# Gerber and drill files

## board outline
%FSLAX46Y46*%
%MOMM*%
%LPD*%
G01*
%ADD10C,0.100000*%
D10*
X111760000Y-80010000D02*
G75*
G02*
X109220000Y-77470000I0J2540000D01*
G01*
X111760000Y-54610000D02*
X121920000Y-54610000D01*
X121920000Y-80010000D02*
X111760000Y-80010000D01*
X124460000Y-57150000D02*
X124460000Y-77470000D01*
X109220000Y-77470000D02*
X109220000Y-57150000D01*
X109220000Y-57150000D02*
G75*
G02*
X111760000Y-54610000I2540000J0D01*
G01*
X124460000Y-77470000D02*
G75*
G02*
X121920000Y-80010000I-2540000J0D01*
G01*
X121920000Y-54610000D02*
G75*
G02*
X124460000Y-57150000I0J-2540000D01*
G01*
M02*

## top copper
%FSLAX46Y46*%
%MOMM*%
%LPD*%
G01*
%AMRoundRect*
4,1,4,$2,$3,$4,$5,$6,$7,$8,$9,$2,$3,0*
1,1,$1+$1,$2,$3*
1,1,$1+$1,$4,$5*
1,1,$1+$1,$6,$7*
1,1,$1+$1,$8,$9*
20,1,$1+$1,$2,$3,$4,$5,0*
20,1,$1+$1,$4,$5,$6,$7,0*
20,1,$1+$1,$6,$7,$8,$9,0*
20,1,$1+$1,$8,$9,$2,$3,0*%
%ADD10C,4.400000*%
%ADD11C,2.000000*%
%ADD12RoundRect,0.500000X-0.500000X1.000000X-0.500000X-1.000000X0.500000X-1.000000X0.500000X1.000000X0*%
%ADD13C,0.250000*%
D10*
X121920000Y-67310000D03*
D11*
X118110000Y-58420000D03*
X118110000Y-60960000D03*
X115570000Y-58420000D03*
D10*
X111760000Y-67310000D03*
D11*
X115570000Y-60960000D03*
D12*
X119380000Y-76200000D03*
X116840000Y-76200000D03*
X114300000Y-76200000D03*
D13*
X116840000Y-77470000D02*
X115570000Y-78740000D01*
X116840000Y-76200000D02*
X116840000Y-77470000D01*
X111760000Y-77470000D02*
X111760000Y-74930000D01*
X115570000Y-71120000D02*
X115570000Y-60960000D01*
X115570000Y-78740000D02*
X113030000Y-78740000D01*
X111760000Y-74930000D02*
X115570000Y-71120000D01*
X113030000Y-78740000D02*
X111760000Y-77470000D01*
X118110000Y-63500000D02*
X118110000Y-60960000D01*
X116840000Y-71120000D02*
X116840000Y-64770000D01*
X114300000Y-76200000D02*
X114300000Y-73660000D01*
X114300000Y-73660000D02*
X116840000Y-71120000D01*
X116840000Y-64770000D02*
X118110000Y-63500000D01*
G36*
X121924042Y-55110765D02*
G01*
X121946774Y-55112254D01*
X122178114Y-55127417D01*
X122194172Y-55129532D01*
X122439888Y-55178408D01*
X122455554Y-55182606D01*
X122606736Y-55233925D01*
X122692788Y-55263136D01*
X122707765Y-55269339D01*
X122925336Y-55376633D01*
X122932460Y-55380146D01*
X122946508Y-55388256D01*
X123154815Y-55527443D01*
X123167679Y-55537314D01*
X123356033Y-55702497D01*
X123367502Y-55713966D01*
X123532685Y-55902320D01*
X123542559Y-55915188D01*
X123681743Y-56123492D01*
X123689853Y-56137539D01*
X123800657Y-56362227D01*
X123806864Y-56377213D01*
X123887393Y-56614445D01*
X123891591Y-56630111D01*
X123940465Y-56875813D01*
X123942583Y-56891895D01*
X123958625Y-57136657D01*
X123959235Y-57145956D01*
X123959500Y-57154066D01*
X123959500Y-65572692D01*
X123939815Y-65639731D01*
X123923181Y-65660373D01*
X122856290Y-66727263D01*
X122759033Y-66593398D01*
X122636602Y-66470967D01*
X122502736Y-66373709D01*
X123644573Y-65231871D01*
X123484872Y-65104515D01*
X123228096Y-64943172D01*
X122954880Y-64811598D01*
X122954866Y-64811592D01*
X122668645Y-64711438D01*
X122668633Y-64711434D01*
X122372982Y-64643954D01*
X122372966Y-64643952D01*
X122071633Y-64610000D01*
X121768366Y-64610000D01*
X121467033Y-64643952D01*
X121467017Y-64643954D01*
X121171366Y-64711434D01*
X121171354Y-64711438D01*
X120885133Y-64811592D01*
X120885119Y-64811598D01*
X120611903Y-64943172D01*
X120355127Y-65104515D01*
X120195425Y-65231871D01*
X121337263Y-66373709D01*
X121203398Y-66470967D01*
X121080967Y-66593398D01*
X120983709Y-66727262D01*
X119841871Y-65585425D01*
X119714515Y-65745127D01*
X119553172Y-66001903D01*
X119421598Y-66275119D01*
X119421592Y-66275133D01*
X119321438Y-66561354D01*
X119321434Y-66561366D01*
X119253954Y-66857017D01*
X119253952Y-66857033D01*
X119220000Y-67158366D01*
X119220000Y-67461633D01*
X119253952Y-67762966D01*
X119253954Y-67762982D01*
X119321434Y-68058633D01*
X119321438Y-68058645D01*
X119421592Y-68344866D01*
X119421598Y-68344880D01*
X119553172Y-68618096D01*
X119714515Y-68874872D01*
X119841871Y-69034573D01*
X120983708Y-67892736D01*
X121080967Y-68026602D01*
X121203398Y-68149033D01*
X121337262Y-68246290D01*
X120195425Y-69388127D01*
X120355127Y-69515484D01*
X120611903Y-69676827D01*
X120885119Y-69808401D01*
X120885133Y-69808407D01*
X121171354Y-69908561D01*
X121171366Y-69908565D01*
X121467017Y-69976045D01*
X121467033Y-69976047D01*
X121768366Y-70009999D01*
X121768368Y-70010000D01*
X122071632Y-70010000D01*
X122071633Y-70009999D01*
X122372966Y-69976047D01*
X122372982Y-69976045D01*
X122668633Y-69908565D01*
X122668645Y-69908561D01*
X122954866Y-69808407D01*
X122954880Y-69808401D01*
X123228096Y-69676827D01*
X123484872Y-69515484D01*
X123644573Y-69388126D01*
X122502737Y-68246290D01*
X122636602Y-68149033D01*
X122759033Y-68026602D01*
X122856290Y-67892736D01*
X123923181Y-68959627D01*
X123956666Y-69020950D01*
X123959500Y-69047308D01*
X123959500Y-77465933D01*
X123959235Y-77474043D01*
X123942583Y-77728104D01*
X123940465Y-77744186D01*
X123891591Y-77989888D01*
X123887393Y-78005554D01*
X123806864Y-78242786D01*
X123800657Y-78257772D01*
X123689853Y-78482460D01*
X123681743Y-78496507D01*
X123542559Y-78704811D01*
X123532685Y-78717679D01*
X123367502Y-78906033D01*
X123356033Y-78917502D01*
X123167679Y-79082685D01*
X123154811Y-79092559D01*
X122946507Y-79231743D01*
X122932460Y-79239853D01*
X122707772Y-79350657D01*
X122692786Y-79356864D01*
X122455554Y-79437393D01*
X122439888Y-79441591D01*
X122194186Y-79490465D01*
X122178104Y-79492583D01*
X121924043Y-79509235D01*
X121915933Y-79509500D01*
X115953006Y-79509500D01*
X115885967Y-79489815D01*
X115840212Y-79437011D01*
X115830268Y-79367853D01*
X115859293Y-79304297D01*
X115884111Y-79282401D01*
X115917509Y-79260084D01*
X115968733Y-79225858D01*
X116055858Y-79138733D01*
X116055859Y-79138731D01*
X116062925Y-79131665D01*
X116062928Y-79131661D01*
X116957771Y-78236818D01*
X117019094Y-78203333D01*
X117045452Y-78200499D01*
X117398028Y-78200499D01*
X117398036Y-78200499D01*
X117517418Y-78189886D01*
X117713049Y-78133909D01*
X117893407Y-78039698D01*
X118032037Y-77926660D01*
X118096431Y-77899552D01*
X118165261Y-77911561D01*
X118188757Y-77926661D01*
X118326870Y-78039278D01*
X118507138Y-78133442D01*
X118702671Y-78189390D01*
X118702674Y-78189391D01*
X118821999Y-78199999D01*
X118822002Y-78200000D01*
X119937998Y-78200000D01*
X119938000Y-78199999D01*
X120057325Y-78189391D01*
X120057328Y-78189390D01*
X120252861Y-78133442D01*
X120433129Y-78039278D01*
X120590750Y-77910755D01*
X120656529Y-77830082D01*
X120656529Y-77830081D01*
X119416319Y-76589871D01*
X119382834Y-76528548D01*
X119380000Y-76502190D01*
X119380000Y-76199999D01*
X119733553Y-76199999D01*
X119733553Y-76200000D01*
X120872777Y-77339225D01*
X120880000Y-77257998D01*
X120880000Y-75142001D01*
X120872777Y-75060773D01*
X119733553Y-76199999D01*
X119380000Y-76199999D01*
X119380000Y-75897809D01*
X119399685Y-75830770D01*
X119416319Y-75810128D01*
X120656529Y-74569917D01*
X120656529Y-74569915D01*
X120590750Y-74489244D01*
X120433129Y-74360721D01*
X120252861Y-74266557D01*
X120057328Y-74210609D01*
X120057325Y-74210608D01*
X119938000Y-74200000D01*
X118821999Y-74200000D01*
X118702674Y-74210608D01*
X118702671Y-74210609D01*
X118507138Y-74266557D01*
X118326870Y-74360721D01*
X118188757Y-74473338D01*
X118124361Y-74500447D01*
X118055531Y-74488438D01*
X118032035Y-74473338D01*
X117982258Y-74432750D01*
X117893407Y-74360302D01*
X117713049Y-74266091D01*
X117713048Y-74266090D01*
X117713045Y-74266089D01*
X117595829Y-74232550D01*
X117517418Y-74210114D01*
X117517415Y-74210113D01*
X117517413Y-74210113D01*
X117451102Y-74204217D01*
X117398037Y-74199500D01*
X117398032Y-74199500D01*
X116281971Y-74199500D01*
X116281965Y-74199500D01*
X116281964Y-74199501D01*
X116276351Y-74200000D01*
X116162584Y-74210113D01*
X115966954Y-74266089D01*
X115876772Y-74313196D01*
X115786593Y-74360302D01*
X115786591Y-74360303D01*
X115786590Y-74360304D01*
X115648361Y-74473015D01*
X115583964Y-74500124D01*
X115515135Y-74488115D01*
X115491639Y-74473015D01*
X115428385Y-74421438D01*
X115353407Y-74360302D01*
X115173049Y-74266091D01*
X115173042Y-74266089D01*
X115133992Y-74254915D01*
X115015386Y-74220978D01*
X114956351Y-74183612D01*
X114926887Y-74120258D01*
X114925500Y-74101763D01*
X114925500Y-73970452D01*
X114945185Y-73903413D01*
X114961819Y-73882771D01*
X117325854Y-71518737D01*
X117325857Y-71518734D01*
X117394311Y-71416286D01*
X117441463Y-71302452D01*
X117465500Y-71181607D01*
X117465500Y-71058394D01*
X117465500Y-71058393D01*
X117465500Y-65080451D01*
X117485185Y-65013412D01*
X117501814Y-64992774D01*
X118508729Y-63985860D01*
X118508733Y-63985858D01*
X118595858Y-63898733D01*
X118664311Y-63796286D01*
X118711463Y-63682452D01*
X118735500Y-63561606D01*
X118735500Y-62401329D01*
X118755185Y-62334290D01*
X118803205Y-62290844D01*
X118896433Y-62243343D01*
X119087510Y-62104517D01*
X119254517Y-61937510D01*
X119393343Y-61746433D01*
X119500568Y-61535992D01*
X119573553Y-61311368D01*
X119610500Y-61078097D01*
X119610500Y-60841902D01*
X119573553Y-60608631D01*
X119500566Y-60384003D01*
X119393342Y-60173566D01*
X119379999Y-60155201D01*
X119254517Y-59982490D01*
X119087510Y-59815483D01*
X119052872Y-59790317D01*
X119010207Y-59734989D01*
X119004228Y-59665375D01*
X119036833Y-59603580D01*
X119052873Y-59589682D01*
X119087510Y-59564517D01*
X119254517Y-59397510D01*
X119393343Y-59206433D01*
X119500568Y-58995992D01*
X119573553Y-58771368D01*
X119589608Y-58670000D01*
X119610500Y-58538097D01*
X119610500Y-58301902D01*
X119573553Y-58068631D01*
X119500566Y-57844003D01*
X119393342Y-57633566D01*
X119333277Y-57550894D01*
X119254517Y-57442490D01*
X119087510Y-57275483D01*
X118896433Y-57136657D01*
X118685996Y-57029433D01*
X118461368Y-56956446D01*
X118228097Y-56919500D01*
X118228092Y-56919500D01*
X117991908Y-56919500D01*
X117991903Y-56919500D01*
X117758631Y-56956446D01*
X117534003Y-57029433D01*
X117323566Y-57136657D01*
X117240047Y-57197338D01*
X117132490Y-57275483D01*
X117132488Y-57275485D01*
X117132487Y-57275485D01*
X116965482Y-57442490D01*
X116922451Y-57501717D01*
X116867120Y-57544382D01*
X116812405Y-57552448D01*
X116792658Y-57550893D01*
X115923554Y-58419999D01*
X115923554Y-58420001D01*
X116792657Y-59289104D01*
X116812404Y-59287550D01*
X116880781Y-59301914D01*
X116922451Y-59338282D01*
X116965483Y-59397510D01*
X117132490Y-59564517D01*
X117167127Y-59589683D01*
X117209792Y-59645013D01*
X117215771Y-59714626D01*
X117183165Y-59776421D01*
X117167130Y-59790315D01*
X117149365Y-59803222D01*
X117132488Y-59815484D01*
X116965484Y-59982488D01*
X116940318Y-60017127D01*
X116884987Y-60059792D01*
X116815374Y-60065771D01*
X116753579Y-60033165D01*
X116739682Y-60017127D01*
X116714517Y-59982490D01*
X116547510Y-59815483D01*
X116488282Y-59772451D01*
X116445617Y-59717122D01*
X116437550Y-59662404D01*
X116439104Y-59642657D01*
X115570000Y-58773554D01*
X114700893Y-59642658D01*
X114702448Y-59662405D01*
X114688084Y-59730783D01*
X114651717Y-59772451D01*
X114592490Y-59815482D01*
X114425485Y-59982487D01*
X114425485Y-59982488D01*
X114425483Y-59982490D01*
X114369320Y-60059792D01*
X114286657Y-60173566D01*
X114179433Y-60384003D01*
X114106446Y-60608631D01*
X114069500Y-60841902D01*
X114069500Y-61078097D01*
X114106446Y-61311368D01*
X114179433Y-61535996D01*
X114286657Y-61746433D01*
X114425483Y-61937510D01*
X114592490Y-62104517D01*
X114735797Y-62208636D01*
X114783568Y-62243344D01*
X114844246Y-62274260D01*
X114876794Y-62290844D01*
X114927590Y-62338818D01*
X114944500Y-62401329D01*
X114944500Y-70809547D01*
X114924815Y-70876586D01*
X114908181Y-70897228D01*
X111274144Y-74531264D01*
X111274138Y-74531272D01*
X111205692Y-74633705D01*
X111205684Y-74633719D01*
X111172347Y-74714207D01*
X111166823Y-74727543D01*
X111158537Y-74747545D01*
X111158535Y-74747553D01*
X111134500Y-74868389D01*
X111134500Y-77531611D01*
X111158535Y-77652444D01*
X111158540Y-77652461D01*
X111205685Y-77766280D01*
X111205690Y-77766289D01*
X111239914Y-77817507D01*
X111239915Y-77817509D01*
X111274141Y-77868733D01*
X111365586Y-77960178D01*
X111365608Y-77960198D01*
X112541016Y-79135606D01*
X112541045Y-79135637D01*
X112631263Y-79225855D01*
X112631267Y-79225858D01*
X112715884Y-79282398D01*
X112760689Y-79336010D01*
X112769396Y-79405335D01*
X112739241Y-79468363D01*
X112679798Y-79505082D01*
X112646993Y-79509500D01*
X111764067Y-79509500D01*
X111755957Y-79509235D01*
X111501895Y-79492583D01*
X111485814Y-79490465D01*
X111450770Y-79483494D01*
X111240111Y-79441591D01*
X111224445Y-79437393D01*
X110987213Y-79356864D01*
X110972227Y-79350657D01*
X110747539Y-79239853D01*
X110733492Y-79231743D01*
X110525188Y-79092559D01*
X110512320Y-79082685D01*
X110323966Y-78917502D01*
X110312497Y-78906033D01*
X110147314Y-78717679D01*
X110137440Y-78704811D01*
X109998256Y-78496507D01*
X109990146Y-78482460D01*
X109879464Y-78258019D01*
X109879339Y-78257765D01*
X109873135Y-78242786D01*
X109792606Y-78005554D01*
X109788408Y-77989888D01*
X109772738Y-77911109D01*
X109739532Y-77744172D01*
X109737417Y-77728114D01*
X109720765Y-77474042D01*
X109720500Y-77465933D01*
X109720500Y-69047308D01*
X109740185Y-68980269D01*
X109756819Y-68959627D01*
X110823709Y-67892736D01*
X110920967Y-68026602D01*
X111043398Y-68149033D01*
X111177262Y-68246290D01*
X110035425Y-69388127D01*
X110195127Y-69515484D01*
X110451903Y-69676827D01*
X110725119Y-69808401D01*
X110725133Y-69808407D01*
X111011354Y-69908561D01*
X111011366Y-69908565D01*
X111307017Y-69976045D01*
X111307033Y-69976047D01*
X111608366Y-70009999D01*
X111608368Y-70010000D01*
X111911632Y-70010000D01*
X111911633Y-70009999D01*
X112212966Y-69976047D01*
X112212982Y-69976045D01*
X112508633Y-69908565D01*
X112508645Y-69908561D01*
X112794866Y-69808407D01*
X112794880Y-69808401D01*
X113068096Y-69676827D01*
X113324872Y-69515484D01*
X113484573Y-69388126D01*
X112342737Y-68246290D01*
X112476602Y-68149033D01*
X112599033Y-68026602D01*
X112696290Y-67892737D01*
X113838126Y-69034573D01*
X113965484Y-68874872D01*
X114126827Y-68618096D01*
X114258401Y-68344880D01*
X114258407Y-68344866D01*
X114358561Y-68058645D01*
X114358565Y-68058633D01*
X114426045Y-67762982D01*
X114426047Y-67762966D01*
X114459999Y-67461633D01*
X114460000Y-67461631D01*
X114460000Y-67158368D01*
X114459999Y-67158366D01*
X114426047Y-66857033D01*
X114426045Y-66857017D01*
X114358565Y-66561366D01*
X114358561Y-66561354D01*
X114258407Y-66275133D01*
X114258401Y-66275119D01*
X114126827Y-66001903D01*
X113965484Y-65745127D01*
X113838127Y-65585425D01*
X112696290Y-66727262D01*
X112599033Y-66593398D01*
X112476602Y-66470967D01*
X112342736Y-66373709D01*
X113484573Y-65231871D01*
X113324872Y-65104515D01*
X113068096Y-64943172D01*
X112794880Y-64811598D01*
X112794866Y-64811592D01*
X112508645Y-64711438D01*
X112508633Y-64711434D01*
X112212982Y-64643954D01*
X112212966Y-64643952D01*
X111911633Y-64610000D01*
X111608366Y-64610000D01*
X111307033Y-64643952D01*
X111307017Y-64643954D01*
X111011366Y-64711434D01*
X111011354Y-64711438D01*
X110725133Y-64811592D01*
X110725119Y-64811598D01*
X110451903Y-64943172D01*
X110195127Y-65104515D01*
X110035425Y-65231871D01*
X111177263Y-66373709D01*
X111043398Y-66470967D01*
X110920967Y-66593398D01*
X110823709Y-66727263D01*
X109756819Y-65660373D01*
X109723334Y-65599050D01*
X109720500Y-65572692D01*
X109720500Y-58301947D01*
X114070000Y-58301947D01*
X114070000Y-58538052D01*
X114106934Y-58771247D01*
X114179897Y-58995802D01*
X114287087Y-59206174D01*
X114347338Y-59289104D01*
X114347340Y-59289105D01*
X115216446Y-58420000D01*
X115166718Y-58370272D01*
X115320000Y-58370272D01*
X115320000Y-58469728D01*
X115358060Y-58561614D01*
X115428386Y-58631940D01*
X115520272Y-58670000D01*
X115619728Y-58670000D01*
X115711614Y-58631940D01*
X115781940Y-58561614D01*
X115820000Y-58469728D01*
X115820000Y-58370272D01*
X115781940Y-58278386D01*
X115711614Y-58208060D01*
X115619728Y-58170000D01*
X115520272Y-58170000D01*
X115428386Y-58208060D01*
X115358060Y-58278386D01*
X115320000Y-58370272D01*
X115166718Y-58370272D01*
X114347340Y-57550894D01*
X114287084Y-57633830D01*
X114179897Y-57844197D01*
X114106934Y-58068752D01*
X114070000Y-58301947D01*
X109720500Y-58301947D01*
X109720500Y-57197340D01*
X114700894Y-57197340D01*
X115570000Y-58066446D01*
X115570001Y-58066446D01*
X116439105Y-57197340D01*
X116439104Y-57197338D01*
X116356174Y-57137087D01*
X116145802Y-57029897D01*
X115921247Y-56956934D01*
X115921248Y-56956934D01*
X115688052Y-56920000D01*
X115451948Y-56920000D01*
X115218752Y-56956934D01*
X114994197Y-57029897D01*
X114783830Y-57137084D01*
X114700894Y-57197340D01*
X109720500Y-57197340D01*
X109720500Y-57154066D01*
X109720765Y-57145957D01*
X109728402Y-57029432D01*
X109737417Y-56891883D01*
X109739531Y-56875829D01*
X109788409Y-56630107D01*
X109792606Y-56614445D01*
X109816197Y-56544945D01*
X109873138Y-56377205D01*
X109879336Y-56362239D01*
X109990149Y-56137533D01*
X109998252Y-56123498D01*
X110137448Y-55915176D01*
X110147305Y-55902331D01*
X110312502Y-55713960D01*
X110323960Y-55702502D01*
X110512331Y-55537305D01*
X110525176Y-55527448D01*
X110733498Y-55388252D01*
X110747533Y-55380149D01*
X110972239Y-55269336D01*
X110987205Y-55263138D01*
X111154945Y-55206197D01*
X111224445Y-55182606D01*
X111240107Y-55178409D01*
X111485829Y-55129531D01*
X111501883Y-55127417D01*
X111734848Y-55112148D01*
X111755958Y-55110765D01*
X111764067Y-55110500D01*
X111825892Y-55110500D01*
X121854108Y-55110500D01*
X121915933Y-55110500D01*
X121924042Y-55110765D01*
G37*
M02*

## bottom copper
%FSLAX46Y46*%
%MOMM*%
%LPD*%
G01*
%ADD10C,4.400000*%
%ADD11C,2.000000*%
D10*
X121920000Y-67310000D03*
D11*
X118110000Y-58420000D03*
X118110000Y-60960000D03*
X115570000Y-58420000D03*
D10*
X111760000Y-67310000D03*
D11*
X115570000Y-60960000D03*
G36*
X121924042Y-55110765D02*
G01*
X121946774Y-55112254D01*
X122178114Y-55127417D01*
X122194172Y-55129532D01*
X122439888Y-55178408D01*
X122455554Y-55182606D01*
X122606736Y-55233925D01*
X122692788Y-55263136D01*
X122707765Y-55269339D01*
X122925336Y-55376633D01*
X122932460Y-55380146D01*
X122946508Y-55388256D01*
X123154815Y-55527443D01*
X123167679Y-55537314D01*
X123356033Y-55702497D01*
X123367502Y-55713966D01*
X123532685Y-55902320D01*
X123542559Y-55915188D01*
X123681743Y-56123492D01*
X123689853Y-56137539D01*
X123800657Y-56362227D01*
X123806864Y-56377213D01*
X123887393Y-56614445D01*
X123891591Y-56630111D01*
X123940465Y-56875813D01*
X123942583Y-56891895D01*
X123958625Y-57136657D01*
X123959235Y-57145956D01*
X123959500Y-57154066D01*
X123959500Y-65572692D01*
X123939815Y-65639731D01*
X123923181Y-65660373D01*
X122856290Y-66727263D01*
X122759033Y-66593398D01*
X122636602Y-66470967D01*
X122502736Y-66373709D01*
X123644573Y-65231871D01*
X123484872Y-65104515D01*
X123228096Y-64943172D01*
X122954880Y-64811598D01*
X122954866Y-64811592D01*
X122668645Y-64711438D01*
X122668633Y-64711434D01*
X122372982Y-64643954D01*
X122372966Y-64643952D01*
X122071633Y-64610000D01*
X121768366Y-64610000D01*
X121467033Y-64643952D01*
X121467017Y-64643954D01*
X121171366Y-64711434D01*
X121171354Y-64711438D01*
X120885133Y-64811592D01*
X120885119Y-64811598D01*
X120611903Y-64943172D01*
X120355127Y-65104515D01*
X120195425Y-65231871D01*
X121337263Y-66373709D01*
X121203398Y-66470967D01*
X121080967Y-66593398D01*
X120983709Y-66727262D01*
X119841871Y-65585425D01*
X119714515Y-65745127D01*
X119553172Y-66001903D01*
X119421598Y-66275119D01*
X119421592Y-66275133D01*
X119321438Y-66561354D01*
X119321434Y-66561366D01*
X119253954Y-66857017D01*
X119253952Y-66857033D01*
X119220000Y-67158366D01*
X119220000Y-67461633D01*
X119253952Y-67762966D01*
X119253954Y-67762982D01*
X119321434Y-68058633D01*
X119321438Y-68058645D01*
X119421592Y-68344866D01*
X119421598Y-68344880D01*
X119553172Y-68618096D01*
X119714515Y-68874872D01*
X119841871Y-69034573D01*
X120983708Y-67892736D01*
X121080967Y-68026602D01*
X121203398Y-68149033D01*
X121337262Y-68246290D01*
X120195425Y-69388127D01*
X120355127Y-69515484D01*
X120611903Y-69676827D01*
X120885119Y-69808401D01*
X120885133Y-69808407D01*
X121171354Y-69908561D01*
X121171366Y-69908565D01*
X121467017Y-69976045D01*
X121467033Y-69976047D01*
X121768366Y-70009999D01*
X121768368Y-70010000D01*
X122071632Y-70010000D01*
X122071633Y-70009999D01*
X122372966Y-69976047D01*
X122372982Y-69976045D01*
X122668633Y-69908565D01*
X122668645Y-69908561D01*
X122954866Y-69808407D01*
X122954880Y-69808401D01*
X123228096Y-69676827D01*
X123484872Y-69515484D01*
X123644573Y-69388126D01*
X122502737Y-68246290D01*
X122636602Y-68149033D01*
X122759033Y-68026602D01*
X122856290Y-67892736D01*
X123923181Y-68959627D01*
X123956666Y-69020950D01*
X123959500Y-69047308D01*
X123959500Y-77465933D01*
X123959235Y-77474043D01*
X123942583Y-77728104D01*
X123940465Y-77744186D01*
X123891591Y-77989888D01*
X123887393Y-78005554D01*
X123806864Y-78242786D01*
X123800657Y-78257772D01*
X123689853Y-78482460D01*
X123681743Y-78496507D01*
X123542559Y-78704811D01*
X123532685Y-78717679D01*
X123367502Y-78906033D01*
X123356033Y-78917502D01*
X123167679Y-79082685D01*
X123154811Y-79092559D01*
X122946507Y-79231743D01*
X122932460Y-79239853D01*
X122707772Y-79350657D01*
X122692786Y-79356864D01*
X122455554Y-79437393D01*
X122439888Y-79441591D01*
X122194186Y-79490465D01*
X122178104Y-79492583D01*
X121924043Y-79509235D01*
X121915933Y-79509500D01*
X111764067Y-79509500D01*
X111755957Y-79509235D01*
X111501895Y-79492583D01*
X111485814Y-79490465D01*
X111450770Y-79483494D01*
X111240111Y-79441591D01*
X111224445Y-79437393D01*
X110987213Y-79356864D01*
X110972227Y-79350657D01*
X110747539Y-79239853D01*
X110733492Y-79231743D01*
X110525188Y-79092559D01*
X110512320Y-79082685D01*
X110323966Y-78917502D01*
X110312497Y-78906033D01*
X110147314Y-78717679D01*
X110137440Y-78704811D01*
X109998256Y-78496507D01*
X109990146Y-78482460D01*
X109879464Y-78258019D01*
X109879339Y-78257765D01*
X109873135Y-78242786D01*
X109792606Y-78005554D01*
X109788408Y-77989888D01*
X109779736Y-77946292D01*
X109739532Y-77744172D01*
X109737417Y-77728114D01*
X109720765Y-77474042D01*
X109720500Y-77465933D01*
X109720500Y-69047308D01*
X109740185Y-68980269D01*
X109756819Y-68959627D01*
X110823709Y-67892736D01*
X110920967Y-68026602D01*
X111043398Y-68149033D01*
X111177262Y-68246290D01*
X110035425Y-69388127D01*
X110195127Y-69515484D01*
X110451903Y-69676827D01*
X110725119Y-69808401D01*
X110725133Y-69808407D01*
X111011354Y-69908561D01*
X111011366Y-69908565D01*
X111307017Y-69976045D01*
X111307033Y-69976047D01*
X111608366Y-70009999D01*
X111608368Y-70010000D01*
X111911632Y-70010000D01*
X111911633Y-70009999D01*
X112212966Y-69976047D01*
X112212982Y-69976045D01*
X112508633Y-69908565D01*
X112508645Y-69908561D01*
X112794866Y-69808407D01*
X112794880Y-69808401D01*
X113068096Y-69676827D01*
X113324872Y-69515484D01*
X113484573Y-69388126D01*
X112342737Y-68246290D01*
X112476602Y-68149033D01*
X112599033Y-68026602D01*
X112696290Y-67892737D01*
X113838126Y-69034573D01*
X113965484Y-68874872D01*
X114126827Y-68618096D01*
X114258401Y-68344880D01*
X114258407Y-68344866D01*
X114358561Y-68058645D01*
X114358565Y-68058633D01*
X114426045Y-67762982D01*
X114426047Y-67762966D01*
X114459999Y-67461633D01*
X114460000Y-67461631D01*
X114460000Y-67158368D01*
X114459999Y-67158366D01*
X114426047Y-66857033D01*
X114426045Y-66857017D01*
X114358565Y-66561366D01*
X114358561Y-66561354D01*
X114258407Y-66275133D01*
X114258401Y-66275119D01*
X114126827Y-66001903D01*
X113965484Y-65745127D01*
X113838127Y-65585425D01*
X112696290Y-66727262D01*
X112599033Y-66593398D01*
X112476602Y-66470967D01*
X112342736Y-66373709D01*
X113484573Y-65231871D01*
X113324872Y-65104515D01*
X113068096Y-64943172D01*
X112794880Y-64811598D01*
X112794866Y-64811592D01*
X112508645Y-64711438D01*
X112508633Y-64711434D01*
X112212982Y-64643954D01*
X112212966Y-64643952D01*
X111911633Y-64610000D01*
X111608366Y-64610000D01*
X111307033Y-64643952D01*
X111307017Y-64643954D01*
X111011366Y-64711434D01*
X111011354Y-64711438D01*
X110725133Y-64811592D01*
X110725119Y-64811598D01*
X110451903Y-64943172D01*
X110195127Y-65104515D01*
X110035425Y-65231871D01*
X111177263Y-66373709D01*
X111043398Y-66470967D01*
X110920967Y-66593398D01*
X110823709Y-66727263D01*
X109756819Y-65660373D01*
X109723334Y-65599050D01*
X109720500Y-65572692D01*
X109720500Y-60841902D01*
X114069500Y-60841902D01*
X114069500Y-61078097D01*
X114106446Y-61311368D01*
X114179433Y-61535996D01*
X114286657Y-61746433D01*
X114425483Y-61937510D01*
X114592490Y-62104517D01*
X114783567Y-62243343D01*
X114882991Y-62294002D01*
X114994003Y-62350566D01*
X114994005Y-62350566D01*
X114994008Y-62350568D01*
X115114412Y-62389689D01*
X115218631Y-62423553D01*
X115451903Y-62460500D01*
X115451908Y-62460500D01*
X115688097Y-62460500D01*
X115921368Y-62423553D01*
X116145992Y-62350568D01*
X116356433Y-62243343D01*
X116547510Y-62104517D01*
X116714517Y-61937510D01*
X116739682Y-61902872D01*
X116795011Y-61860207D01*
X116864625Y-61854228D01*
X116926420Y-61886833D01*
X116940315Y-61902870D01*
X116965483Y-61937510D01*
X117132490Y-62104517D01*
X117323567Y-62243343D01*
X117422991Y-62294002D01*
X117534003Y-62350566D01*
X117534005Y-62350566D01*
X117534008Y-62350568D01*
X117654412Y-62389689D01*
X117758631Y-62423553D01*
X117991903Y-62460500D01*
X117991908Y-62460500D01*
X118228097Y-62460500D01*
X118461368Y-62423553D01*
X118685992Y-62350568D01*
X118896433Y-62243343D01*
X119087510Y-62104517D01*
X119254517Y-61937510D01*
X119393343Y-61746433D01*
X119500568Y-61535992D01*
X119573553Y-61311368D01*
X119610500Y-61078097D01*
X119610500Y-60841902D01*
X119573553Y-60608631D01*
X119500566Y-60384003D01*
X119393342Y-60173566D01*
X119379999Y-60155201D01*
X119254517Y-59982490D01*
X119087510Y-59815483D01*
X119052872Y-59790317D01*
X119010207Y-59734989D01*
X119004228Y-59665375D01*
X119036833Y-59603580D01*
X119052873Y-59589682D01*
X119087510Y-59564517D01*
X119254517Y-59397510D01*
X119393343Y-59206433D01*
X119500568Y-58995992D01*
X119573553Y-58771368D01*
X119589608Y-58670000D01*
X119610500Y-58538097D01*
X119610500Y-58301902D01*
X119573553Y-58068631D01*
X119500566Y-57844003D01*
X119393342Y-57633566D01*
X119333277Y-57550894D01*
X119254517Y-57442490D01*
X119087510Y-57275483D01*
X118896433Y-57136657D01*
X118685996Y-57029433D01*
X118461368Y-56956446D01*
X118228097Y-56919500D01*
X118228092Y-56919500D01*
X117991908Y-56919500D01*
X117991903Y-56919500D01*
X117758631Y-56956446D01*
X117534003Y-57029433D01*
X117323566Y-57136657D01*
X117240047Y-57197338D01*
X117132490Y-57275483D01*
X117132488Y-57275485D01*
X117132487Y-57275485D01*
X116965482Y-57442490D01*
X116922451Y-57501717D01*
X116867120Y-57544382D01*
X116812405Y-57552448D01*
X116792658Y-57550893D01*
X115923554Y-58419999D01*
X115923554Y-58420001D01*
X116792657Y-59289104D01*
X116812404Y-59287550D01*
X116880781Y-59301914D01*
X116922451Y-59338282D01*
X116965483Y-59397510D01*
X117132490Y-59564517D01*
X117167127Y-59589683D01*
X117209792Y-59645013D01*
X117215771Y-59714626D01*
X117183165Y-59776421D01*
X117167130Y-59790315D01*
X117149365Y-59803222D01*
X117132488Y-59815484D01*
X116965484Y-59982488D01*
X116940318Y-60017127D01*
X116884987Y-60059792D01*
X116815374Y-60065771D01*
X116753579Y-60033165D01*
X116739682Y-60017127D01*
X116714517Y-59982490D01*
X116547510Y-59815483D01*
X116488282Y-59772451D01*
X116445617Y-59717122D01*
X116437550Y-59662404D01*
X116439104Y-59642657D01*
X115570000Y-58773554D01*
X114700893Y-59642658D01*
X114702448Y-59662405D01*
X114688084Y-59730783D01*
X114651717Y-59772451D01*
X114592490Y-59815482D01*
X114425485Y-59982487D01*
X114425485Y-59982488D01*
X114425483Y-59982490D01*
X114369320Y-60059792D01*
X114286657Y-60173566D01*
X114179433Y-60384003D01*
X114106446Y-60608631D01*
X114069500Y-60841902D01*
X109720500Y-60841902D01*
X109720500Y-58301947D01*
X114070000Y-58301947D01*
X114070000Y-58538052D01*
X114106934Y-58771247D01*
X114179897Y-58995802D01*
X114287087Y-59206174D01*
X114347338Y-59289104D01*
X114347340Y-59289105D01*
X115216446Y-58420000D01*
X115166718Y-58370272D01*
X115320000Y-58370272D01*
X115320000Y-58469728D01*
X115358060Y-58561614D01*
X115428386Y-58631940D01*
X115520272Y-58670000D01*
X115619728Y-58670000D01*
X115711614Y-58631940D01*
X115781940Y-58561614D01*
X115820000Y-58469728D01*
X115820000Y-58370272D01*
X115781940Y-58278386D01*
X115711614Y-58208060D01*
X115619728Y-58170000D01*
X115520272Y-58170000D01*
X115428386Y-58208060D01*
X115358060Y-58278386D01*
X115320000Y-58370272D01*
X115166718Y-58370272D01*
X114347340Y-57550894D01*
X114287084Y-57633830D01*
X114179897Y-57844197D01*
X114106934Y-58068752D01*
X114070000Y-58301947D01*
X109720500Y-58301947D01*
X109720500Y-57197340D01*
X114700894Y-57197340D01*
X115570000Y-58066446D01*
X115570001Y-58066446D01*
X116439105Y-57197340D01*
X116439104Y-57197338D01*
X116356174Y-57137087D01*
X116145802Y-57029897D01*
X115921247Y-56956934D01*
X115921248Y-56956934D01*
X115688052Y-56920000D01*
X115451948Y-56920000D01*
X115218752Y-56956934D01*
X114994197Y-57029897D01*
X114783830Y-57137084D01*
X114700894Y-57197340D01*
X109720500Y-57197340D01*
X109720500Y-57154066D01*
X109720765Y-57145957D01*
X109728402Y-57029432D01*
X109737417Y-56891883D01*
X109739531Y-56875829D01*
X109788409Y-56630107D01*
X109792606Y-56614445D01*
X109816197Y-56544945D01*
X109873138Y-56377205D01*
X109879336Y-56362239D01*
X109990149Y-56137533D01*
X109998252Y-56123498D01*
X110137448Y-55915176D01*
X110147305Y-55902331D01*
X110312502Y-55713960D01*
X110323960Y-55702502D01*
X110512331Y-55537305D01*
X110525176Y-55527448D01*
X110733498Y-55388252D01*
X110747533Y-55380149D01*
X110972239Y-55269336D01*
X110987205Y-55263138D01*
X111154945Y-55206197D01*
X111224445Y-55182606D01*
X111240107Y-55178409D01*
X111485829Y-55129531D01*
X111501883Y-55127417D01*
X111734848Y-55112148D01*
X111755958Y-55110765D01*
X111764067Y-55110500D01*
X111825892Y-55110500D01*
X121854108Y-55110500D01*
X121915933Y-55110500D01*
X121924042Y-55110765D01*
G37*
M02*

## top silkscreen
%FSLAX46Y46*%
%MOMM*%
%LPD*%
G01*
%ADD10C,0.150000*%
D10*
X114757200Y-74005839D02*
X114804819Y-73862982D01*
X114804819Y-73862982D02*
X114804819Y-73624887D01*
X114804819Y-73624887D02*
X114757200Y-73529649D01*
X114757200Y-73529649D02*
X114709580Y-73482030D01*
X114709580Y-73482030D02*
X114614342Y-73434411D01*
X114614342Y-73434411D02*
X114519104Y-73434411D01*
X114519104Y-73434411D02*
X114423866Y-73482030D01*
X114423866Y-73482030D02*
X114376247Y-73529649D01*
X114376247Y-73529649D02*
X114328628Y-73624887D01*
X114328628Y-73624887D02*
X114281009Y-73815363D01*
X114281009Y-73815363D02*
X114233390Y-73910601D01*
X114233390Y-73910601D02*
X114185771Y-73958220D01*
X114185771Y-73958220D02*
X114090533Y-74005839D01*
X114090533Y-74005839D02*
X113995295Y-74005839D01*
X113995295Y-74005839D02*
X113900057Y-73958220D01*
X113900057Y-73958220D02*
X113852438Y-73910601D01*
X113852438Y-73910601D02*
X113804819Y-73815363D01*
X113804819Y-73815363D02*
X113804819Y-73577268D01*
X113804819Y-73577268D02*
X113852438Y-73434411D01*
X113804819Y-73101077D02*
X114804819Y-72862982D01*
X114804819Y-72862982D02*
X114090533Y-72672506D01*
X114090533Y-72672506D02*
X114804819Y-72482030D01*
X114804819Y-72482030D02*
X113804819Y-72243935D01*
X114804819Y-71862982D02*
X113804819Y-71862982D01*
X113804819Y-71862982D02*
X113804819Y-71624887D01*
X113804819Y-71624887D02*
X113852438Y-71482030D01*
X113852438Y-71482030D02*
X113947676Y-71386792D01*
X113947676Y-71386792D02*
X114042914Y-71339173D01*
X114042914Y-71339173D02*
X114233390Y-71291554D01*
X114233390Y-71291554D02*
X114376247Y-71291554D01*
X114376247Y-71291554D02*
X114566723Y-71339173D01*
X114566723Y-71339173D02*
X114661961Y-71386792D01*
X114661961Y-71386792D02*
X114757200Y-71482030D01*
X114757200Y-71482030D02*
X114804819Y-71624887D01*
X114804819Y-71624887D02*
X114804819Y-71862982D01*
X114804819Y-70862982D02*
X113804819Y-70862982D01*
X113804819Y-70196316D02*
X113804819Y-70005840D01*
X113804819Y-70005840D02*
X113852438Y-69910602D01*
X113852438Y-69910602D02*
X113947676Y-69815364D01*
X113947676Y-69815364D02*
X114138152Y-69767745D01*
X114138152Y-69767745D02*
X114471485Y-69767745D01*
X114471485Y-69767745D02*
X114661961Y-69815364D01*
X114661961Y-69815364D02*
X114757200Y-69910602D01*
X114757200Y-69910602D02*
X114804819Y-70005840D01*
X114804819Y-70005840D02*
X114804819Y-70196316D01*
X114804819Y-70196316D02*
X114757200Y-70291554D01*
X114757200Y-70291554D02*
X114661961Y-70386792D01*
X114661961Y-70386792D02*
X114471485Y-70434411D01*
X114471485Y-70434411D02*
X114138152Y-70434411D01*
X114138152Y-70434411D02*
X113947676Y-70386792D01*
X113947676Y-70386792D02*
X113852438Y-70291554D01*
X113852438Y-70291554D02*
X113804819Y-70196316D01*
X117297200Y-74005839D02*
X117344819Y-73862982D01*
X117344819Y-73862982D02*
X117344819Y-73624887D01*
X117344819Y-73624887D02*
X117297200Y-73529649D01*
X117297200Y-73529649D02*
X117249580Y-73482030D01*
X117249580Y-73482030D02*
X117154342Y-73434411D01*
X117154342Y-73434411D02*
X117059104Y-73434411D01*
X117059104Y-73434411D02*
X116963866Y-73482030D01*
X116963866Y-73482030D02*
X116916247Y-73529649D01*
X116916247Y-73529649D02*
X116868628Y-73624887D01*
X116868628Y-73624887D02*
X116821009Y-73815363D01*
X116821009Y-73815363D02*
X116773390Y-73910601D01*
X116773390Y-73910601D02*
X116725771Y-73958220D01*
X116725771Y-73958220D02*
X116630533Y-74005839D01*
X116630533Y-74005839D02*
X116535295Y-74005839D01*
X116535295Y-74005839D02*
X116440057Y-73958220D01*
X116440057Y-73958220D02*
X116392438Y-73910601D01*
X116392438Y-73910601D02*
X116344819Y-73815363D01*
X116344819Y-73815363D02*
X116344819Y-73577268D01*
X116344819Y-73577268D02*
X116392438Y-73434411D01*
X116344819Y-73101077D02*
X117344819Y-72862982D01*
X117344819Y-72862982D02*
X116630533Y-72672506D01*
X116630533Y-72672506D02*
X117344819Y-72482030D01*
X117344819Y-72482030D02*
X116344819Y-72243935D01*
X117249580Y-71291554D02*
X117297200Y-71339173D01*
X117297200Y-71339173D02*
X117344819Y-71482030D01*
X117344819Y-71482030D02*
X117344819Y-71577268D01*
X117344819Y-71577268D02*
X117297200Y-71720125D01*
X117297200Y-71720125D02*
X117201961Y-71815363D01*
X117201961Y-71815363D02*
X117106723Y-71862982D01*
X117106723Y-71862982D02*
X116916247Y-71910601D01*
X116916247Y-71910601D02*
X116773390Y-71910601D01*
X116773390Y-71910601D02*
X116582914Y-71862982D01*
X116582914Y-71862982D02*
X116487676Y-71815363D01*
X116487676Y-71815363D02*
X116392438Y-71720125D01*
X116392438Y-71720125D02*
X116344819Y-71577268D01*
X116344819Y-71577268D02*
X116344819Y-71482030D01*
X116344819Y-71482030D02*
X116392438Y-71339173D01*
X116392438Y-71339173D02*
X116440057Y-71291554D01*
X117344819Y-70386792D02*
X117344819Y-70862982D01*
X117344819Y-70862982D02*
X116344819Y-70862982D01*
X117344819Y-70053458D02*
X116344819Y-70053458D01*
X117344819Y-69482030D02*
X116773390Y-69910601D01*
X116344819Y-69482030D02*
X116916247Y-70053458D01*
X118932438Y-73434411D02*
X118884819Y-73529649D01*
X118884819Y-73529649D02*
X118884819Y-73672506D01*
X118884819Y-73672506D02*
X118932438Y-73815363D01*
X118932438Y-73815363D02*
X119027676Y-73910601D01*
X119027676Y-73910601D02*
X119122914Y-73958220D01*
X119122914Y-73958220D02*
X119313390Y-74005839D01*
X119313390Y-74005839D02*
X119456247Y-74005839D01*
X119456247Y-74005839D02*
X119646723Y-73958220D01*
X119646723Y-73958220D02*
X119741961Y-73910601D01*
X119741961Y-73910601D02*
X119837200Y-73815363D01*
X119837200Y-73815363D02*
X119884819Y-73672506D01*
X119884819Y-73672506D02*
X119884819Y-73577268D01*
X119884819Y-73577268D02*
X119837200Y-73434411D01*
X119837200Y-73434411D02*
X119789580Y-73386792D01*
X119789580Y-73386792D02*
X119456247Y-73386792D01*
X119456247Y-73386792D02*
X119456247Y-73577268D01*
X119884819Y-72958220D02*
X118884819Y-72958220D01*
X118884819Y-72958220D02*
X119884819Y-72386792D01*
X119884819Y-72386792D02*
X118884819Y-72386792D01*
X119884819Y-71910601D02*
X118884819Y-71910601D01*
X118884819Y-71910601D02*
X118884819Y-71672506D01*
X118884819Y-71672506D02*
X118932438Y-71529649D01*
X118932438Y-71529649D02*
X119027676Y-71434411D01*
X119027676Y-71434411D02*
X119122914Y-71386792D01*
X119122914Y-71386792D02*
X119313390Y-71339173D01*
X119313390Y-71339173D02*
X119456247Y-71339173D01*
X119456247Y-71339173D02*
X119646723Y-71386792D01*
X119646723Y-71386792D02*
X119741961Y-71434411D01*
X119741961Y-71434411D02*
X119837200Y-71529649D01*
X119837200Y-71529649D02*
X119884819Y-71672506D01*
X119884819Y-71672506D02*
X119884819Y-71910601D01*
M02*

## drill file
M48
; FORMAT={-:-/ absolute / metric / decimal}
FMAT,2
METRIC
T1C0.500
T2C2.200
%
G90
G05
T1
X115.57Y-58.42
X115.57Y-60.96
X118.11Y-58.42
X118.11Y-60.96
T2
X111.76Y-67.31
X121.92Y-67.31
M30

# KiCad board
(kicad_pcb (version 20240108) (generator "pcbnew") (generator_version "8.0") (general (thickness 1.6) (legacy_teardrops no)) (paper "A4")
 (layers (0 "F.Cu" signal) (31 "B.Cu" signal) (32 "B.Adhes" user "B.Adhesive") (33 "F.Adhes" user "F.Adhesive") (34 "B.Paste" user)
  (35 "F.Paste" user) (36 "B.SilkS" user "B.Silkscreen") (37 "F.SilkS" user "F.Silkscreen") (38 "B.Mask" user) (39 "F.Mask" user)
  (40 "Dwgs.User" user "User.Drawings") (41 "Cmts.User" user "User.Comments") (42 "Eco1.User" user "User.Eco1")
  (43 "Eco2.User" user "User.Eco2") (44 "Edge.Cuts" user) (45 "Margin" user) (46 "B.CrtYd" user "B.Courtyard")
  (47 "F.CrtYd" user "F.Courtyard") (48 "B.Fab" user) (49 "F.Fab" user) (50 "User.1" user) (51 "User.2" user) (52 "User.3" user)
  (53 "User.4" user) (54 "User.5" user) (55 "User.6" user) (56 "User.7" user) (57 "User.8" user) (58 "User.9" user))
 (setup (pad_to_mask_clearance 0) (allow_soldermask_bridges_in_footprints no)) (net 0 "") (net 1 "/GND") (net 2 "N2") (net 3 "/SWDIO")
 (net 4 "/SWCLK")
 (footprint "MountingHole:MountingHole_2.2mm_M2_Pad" (layer "F.Cu") (at 121.92 67.31)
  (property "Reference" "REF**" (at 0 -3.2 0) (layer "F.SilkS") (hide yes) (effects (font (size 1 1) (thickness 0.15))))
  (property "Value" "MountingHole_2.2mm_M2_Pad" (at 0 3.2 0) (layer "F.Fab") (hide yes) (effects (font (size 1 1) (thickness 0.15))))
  (pad "1" thru_hole circle (at 0 0) (size 4.4 4.4) (drill 2.2) (layers "*.Cu" "*.Mask") (remove_unused_layers no) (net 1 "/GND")))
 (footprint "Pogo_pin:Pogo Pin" (layer "F.Cu") (at 118.11 58.42)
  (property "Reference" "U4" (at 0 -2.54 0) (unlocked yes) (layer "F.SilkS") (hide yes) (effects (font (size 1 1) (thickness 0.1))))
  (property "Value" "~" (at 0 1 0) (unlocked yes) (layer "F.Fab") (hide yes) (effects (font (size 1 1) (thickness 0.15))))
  (pad "1" thru_hole circle (at 0 0) (size 2 2) (drill 0.5) (layers "*.Cu" "*.Mask") (remove_unused_layers no) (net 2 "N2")))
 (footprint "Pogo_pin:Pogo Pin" (layer "F.Cu") (at 118.11 60.96)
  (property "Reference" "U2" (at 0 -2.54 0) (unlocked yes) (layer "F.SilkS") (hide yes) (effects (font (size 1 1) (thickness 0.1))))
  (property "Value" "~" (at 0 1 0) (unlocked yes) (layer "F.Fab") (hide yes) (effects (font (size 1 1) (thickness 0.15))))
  (pad "1" thru_hole circle (at 0 0) (size 2 2) (drill 0.5) (layers "*.Cu" "*.Mask") (remove_unused_layers no) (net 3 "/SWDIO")))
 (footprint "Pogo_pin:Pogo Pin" (layer "F.Cu") (at 115.57 58.42)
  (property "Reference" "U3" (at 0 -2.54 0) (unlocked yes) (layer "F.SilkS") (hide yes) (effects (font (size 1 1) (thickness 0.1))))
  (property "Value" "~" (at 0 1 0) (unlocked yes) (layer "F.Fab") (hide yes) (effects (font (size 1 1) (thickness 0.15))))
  (pad "1" thru_hole circle (at 0 0) (size 2 2) (drill 0.5) (layers "*.Cu" "*.Mask") (remove_unused_layers no) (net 1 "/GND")))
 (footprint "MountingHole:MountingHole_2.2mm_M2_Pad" (layer "F.Cu") (at 111.76 67.31)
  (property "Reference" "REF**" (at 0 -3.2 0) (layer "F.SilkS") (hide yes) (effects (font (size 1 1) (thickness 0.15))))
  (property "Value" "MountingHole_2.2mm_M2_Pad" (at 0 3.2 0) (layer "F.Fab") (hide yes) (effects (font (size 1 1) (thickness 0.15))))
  (pad "1" thru_hole circle (at 0 0) (size 4.4 4.4) (drill 2.2) (layers "*.Cu" "*.Mask") (remove_unused_layers no) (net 1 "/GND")))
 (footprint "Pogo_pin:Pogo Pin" (layer "F.Cu") (at 115.57 60.96)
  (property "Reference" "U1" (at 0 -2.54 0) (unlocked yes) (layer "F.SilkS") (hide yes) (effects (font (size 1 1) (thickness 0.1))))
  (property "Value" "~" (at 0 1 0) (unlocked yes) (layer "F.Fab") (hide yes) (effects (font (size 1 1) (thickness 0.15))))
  (pad "1" thru_hole circle (at 0 0) (size 2 2) (drill 0.5) (layers "*.Cu" "*.Mask") (remove_unused_layers no) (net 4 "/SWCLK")))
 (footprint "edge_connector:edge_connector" (layer "F.Cu") (at 116.84 76.2 -90)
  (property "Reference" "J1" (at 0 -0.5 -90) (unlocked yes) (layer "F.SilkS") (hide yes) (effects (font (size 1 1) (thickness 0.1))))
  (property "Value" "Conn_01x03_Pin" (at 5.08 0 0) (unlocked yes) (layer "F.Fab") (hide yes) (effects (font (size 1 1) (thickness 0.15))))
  (pad "1" smd roundrect (at 0 -2.54 270) (size 3 2) (layers "F.Cu" "F.Mask") (roundrect_rratio 0.25) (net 1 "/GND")
   (thermal_bridge_angle 45))
  (pad "2" smd roundrect (at 0 0 270) (size 3 2) (layers "F.Cu" "F.Mask") (roundrect_rratio 0.25) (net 4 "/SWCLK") (thermal_bridge_angle 45))
  (pad "3" smd roundrect (at 0 2.54 270) (size 3 2) (layers "F.Cu" "F.Mask") (roundrect_rratio 0.25) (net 3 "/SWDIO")
   (thermal_bridge_angle 45)))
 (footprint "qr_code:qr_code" (layer "B.Cu") (at 116.84 74.93 180)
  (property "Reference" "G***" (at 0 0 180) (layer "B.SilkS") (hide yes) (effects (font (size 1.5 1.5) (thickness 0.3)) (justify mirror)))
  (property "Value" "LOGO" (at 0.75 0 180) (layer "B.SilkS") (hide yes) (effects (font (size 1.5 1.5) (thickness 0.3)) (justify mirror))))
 (gr_arc (start 111.76 80.01) (mid 109.963949 79.266051) (end 109.22 77.47) (stroke (width 0.1) (type default)) (layer "Edge.Cuts"))
 (gr_line (start 111.76 54.61) (end 121.92 54.61) (stroke (width 0.1) (type default)) (layer "Edge.Cuts"))
 (gr_line (start 121.92 80.01) (end 111.76 80.01) (stroke (width 0.1) (type default)) (layer "Edge.Cuts"))
 (gr_line (start 124.46 57.15) (end 124.46 77.47) (stroke (width 0.1) (type default)) (layer "Edge.Cuts"))
 (gr_line (start 109.22 77.47) (end 109.22 57.15) (stroke (width 0.1) (type default)) (layer "Edge.Cuts"))
 (gr_arc (start 109.22 57.15) (mid 109.963949 55.353949) (end 111.76 54.61) (stroke (width 0.1) (type default)) (layer "Edge.Cuts"))
 (gr_arc (start 124.46 77.47) (mid 123.716051 79.266051) (end 121.92 80.01) (stroke (width 0.1) (type default)) (layer "Edge.Cuts"))
 (gr_arc (start 121.92 54.61) (mid 123.716051 55.353949) (end 124.46 57.15) (stroke (width 0.1) (type default)) (layer "Edge.Cuts"))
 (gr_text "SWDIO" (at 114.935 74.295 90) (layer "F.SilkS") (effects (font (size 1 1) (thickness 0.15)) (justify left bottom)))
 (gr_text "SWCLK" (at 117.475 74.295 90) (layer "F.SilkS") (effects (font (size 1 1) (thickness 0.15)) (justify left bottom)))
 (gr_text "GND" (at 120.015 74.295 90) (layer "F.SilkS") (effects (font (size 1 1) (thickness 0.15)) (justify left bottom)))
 (segment (start 116.84 77.47) (end 115.57 78.74) (width 0.25) (layer "F.Cu") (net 4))
 (segment (start 116.84 76.2) (end 116.84 77.47) (width 0.25) (layer "F.Cu") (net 4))
 (segment (start 111.76 77.47) (end 111.76 74.93) (width 0.25) (layer "F.Cu") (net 4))
 (segment (start 115.57 71.12) (end 115.57 60.96) (width 0.25) (layer "F.Cu") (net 4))
 (segment (start 115.57 78.74) (end 113.03 78.74) (width 0.25) (layer "F.Cu") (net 4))
 (segment (start 111.76 74.93) (end 115.57 71.12) (width 0.25) (layer "F.Cu") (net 4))
 (segment (start 113.03 78.74) (end 111.76 77.47) (width 0.25) (layer "F.Cu") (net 4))
 (segment (start 118.11 63.5) (end 118.11 60.96) (width 0.25) (layer "F.Cu") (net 3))
 (segment (start 116.84 71.12) (end 116.84 64.77) (width 0.25) (layer "F.Cu") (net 3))
 (segment (start 114.3 76.2) (end 114.3 73.66) (width 0.25) (layer "F.Cu") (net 3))
 (segment (start 114.3 73.66) (end 116.84 71.12) (width 0.25) (layer "F.Cu") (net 3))
 (segment (start 116.84 64.77) (end 118.11 63.5) (width 0.25) (layer "F.Cu") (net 3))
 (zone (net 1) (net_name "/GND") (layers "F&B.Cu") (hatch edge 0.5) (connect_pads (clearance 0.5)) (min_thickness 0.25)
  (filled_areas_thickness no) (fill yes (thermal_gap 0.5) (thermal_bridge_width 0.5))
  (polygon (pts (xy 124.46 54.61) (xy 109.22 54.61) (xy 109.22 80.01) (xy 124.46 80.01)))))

